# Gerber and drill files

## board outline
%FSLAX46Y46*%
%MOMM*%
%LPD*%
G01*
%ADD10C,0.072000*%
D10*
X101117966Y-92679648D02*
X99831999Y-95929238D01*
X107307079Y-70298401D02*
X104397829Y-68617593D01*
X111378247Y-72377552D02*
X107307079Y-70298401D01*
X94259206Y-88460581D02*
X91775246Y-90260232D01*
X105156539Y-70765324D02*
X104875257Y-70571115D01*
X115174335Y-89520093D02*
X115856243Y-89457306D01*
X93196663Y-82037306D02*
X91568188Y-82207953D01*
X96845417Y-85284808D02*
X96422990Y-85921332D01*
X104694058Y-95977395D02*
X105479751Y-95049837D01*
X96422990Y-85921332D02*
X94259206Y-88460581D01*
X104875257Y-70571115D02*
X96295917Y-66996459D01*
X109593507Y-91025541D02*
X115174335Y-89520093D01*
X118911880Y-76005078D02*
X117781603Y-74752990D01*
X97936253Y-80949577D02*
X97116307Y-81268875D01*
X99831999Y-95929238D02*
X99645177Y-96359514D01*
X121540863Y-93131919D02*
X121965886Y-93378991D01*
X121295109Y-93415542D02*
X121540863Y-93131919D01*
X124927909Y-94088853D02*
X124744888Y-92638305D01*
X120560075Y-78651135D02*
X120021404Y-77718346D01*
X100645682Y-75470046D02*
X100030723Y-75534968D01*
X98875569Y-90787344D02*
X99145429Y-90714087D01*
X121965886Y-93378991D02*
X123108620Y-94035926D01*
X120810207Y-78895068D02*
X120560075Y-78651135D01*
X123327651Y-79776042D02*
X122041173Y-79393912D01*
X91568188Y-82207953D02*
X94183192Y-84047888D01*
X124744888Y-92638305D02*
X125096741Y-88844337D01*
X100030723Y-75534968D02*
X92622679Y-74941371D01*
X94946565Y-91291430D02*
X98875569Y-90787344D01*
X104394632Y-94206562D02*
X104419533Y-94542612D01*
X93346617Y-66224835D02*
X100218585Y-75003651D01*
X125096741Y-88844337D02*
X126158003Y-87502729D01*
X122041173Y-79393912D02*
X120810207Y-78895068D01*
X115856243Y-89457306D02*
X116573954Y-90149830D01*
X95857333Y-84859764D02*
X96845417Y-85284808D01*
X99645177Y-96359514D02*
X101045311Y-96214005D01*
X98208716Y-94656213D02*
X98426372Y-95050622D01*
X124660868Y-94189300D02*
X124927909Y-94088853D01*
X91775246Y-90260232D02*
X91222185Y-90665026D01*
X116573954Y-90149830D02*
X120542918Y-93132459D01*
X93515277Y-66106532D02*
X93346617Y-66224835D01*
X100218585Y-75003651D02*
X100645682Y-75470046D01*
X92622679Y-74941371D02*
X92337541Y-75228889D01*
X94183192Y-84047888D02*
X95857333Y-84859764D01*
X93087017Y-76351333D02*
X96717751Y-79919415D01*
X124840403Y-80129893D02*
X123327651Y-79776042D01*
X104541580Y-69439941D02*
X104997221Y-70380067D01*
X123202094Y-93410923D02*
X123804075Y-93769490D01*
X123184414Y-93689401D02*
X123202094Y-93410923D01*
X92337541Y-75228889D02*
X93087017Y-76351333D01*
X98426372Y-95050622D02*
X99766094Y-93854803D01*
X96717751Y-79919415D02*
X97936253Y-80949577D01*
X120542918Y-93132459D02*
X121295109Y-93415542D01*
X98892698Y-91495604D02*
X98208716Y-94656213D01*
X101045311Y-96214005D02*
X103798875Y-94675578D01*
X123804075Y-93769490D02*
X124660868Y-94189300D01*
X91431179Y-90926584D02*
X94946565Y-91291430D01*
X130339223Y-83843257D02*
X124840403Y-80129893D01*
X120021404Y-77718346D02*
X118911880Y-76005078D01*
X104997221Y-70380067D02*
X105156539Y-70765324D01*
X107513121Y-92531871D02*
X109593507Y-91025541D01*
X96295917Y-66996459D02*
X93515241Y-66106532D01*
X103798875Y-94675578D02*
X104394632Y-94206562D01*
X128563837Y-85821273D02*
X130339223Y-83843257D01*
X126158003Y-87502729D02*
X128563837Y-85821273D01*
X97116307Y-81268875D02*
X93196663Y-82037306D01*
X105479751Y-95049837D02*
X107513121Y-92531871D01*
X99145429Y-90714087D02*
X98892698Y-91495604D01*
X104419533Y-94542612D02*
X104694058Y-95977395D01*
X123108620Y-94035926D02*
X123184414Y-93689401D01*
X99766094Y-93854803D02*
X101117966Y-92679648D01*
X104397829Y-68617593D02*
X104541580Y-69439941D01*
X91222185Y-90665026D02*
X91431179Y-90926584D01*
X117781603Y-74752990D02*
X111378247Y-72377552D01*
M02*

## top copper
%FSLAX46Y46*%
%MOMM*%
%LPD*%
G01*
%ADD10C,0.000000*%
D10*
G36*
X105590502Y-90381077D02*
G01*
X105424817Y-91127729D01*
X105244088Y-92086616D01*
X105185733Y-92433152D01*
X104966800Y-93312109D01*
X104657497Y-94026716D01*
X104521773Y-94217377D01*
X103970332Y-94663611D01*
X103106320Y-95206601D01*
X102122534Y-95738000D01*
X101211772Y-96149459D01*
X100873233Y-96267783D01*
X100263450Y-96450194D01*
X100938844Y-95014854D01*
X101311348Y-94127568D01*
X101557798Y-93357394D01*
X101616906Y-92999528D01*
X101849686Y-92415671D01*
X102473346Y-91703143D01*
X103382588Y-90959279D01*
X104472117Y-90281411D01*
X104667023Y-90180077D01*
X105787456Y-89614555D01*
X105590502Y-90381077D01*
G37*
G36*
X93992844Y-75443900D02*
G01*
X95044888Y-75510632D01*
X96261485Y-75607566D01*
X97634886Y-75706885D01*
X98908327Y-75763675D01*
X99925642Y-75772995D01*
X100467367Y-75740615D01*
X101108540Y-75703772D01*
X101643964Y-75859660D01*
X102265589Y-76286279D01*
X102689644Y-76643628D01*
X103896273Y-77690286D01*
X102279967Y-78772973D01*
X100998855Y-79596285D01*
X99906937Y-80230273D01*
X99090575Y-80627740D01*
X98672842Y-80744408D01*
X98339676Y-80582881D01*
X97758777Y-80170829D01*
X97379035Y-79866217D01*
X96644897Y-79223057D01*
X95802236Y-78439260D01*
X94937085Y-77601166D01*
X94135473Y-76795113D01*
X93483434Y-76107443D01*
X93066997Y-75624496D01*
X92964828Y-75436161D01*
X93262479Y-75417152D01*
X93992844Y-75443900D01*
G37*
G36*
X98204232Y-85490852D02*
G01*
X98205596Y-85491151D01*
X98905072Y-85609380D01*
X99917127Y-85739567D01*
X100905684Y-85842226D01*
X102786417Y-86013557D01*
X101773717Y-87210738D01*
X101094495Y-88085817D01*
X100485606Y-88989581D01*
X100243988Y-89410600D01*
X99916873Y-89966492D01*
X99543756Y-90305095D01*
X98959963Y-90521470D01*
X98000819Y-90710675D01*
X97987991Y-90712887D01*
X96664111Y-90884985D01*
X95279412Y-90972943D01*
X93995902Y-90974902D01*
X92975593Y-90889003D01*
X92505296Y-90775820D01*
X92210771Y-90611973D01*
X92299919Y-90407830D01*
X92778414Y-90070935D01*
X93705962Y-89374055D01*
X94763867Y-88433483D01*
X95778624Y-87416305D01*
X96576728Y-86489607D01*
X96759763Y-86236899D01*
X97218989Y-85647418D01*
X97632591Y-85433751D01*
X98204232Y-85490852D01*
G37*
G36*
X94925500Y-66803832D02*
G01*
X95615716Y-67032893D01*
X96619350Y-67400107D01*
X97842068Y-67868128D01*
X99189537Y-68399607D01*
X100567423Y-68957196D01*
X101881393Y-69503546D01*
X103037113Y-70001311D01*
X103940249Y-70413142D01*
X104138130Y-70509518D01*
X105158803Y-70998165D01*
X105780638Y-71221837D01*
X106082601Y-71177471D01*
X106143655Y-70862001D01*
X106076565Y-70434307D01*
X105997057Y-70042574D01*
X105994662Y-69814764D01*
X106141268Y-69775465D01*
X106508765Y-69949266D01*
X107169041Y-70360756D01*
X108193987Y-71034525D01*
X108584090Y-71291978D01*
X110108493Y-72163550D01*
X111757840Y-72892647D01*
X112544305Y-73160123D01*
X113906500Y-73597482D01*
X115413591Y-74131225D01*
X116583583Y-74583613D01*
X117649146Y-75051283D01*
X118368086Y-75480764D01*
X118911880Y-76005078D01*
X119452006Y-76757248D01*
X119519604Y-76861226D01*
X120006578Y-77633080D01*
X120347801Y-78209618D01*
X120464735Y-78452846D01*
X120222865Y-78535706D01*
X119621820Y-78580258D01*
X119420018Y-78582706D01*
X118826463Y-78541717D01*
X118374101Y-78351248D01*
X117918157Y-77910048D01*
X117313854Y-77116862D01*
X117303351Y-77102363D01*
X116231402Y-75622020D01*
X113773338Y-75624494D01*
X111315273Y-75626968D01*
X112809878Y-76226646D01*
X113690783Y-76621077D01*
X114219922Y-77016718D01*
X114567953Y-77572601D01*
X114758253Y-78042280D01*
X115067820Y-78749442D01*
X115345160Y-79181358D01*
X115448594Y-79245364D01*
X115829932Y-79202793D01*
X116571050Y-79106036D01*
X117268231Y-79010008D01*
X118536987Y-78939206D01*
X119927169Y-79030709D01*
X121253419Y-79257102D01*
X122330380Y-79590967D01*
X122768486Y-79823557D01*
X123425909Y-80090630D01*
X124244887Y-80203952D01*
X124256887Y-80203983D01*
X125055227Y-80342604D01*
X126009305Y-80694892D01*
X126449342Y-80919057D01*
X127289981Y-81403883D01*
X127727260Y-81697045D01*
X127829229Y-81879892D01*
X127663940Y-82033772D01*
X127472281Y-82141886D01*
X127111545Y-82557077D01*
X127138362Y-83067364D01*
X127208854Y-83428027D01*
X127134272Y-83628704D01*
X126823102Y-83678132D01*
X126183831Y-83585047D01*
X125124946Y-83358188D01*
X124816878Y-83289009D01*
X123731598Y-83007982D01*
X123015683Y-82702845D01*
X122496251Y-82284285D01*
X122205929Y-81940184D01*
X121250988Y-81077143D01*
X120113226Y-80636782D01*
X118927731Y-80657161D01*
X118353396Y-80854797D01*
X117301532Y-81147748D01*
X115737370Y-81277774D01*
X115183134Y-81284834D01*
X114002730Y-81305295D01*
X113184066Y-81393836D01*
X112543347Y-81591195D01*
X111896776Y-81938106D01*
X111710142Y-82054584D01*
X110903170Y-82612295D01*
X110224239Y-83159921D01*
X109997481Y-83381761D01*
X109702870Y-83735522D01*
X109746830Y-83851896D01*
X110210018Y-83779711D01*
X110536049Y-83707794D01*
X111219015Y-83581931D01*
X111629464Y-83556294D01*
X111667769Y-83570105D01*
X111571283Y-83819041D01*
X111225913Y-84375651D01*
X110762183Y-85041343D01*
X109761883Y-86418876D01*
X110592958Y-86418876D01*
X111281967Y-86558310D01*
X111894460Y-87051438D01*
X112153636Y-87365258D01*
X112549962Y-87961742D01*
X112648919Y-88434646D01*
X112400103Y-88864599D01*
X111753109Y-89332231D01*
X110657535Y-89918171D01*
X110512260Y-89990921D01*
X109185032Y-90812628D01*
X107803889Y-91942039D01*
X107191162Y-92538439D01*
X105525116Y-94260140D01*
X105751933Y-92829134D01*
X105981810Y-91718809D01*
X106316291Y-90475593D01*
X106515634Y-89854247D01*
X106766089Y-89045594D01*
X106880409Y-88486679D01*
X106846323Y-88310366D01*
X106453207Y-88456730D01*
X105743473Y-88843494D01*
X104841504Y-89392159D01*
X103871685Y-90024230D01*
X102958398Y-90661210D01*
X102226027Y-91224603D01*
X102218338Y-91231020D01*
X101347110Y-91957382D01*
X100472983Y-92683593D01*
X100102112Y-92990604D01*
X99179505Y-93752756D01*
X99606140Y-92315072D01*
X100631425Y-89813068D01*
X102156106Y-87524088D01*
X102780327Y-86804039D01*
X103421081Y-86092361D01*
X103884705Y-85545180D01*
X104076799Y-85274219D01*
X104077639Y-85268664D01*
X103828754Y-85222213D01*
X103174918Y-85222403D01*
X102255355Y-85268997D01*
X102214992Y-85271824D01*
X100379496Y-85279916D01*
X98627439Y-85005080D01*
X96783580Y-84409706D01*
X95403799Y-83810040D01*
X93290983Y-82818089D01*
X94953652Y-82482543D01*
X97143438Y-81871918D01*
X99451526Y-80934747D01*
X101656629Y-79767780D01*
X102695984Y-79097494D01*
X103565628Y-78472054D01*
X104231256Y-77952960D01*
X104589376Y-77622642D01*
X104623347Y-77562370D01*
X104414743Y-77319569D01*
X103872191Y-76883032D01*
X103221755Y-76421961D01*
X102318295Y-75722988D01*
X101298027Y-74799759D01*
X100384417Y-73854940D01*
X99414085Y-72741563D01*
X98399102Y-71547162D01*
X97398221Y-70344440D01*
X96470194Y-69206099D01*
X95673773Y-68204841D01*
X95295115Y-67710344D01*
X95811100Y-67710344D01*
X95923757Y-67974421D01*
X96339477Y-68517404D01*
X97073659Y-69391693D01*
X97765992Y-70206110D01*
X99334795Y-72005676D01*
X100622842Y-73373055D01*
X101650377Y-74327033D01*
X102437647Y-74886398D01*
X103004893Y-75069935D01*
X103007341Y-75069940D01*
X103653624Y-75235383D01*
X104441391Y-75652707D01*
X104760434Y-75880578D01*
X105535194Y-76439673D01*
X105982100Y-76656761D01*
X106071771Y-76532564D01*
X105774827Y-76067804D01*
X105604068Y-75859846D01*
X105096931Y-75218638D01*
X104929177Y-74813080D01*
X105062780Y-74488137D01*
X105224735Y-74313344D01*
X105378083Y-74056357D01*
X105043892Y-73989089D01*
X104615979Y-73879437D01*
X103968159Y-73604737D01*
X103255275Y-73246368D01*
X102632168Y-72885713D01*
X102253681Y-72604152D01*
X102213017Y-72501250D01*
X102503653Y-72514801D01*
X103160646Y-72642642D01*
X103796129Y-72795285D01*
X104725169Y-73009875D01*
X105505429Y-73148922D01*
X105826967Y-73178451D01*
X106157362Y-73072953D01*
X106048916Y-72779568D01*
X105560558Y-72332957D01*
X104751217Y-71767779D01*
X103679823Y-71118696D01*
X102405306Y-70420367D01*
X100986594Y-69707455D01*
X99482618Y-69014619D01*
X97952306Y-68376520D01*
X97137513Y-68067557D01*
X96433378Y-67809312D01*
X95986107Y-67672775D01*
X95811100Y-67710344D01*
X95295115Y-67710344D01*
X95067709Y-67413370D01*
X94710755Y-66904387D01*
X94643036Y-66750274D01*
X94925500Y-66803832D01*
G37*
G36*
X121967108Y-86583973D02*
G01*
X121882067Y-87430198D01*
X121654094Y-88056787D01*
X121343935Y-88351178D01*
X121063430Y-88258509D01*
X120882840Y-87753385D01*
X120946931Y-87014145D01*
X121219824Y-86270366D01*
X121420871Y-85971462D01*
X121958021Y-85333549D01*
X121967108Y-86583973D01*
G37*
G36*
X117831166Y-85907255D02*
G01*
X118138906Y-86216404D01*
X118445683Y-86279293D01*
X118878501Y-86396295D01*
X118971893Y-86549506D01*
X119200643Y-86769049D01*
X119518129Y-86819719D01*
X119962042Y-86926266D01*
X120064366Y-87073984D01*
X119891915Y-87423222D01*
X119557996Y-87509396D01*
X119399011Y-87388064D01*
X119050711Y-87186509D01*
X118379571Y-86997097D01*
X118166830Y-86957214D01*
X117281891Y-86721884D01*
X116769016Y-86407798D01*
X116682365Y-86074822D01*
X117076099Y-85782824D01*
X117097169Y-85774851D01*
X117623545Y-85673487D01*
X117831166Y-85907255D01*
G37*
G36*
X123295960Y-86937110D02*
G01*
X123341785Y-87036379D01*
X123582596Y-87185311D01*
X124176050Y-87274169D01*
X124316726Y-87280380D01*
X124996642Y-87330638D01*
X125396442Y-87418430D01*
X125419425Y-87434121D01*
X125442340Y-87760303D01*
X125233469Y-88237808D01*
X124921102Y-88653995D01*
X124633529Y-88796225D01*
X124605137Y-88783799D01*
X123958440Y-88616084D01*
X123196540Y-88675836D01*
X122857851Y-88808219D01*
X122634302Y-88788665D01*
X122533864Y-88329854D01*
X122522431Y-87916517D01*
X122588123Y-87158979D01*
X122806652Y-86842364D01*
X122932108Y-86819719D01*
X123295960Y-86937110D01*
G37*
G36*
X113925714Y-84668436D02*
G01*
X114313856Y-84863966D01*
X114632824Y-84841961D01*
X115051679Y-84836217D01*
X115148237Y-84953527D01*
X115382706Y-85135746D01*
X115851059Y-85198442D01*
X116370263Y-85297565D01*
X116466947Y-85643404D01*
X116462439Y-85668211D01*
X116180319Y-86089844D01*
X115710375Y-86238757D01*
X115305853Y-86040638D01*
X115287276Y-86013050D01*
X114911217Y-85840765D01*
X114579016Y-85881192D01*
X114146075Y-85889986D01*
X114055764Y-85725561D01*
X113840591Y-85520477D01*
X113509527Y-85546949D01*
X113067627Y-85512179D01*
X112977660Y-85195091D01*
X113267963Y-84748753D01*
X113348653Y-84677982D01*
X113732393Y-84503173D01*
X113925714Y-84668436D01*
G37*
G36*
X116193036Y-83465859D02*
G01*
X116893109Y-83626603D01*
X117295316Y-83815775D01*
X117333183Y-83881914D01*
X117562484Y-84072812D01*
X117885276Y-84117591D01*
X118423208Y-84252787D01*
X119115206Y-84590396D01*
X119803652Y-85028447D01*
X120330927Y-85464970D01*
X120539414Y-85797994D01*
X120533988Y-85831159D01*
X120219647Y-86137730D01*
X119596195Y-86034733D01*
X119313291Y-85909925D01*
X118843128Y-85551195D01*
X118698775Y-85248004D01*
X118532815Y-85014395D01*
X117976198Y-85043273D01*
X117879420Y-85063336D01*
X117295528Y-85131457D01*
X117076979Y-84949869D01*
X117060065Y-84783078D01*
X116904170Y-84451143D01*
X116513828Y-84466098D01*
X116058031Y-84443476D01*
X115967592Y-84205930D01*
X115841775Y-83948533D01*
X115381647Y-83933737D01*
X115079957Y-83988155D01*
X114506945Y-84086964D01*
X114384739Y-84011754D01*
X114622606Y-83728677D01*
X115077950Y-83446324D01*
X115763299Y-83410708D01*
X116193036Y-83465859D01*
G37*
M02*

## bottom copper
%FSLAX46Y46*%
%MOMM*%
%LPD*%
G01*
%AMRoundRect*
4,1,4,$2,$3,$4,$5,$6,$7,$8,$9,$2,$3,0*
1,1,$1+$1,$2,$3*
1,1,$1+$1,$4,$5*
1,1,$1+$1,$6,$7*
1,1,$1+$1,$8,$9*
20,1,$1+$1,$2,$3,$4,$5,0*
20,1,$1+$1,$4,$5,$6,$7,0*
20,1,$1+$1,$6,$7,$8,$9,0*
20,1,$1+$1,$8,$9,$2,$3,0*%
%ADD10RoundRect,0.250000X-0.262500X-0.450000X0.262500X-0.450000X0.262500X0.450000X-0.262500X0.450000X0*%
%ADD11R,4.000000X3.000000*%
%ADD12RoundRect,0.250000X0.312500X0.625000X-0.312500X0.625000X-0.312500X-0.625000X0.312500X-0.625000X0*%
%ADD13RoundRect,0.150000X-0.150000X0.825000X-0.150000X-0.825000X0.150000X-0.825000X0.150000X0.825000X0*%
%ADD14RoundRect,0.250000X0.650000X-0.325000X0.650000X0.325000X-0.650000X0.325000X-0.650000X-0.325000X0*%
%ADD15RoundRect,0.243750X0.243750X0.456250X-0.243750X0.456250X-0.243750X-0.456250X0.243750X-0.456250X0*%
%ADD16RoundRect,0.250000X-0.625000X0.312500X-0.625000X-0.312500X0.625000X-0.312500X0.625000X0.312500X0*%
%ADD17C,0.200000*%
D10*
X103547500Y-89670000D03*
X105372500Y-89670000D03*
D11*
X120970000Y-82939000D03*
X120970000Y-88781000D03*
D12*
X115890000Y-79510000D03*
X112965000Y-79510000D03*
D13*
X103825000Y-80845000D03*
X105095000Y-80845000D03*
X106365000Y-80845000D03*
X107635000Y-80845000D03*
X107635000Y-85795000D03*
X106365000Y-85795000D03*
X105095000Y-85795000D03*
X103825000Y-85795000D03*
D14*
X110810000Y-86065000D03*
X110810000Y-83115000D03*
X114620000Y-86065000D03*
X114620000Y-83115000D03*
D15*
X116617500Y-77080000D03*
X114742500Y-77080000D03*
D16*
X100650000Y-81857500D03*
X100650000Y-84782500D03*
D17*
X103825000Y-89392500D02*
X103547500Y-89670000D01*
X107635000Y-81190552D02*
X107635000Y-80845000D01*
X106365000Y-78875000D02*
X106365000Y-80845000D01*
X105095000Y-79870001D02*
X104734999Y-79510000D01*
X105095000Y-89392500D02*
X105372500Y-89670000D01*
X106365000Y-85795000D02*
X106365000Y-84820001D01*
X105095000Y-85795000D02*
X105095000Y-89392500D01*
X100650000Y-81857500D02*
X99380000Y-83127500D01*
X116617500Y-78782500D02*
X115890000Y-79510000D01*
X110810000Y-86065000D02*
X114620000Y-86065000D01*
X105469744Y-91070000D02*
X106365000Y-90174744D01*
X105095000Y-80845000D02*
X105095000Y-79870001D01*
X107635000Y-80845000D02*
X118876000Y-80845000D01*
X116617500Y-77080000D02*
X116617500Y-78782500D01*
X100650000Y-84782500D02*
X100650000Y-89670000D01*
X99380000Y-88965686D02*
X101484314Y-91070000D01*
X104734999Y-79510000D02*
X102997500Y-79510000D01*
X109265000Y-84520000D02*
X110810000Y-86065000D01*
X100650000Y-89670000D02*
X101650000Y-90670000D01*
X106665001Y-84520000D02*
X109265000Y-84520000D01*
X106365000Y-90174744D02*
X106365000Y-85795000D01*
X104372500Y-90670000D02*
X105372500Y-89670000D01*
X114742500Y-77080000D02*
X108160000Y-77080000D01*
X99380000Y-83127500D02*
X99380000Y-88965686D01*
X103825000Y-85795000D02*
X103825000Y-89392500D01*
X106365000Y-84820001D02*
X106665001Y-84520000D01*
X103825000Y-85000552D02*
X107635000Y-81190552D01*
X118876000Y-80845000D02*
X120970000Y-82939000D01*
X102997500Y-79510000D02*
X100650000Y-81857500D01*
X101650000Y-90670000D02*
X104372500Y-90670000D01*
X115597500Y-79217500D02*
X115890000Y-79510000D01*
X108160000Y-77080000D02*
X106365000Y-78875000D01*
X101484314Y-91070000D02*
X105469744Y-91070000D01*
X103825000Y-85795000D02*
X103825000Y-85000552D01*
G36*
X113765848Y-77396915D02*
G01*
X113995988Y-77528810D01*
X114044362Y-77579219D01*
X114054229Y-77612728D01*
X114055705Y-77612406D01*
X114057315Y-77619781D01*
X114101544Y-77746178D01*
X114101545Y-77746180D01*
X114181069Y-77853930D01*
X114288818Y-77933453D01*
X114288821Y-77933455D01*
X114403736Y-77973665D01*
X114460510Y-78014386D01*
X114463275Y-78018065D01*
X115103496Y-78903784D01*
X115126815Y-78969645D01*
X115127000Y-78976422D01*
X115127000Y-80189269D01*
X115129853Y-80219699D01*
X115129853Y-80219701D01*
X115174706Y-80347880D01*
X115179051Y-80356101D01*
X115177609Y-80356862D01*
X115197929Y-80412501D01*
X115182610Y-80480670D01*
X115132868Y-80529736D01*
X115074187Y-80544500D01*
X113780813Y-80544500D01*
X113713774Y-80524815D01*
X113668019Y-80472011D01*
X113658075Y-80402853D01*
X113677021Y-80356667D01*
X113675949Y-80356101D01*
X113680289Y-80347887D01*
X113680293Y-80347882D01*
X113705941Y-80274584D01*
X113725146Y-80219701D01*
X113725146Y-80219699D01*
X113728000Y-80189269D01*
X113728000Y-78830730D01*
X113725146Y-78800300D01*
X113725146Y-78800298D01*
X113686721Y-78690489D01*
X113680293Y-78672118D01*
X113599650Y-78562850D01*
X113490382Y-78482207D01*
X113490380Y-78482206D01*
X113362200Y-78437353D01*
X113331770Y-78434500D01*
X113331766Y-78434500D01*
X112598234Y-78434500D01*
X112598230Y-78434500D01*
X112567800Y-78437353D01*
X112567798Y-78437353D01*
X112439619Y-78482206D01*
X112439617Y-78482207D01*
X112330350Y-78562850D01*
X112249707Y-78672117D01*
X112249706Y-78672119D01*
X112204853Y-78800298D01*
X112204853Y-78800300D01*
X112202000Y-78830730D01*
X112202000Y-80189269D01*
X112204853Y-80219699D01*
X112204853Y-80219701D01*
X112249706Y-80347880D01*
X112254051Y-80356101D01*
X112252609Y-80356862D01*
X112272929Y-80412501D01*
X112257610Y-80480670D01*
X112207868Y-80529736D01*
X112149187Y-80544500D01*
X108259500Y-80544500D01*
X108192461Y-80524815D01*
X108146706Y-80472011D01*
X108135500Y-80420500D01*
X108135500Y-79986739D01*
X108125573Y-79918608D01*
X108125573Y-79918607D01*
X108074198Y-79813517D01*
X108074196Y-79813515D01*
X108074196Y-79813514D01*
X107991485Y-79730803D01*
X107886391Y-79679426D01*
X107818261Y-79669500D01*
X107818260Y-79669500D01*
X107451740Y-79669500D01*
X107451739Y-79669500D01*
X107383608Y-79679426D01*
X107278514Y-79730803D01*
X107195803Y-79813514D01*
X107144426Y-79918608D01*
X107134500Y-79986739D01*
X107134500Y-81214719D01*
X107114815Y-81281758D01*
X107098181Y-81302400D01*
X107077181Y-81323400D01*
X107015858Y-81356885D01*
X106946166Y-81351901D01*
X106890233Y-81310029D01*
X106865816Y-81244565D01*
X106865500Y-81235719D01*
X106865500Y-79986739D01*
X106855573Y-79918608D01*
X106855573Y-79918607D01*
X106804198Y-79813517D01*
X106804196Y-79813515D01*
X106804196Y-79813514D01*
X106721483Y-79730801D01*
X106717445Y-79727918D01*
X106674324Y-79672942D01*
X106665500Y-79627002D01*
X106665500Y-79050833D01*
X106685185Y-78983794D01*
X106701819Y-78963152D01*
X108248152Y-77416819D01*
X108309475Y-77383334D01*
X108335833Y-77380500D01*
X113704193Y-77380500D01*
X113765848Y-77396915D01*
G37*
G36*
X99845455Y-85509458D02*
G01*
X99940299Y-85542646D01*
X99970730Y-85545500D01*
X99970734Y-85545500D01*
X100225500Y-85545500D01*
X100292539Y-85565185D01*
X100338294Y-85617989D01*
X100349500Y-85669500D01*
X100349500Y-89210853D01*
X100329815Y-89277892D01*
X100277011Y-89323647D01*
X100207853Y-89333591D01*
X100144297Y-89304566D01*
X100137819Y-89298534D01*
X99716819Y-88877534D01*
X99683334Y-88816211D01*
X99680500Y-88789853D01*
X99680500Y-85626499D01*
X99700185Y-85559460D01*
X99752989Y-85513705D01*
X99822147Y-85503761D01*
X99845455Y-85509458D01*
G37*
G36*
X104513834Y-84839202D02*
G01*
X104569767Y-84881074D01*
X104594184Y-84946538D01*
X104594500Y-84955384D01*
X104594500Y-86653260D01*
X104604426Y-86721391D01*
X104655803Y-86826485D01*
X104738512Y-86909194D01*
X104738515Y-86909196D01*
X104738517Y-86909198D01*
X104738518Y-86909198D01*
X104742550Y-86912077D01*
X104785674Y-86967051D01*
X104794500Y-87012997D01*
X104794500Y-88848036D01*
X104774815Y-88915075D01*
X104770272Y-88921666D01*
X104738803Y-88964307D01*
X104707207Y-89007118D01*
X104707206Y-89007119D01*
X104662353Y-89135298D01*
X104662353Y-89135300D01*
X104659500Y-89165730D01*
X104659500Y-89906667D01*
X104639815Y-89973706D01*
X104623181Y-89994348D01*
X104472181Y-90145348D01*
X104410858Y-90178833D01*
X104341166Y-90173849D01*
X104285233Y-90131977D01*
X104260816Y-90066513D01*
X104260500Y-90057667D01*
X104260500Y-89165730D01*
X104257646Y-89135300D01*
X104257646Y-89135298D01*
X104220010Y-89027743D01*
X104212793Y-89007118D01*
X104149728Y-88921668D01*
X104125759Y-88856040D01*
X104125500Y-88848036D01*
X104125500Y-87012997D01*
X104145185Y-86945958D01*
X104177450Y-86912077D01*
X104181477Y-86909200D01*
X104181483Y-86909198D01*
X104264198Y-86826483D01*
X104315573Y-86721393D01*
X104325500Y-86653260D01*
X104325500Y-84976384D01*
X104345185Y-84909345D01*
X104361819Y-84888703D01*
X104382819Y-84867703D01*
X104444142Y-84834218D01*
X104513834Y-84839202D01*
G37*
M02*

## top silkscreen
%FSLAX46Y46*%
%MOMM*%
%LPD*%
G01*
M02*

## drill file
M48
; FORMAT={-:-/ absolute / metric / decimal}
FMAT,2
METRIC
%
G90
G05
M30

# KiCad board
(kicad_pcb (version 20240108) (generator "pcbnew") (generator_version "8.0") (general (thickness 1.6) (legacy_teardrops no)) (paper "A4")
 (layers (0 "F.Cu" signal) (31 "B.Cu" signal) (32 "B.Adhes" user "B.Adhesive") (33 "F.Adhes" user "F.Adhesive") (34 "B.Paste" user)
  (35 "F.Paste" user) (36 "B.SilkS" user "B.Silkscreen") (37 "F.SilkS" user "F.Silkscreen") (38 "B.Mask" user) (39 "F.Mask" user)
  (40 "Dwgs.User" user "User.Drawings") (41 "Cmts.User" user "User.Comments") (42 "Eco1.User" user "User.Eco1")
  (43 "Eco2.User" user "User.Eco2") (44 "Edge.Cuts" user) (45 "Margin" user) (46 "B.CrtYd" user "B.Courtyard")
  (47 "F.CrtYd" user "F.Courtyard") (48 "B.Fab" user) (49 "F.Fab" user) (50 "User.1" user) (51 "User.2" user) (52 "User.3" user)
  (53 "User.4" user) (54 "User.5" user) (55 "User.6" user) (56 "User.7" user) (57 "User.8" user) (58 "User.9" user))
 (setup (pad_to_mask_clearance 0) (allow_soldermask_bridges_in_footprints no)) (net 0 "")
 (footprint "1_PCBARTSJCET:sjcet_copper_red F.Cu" (layer "F.Cu") (at 118.552907 138.299727)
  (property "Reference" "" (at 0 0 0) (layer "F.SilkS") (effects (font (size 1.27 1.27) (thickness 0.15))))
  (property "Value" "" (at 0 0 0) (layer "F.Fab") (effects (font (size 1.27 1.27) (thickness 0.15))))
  (fp_poly
   (pts (xy -12.962405 -47.91865) (xy -13.12809 -47.171998) (xy -13.308819 -46.213111) (xy -13.367174 -45.866575) (xy -13.586107 -44.987618)
    (xy -13.89541 -44.273011) (xy -14.031134 -44.08235) (xy -14.582575 -43.636116) (xy -15.446587 -43.093126) (xy -16.430373 -42.561727)
    (xy -17.341135 -42.150268) (xy -17.679674 -42.031944) (xy -18.289457 -41.849533) (xy -17.614063 -43.284873) (xy -17.241559 -44.172159)
    (xy -16.995109 -44.942333) (xy -16.936001 -45.300199) (xy -16.703221 -45.884056) (xy -16.079561 -46.596584) (xy -15.170319 -47.340448)
    (xy -14.08079 -48.018316) (xy -13.885884 -48.11965) (xy -12.765451 -48.685172))
   (stroke (width 0) (type solid)) (fill solid) (layer "F.Cu"))
  (fp_poly
   (pts (xy -24.560063 -62.855827) (xy -23.508019 -62.789095) (xy -22.291422 -62.692161) (xy -20.918021 -62.592842)
    (xy -19.64458 -62.536052) (xy -18.627265 -62.526732) (xy -18.08554 -62.559112) (xy -17.444367 -62.595955) (xy -16.908943 -62.440067)
    (xy -16.287318 -62.013448) (xy -15.863263 -61.656099) (xy -14.656634 -60.609441) (xy -16.27294 -59.526754) (xy -17.554052 -58.703442)
    (xy -18.64597 -58.069454) (xy -19.462332 -57.671987) (xy -19.880065 -57.555319) (xy -20.213231 -57.716846) (xy -20.79413 -58.128898)
    (xy -21.173872 -58.43351) (xy -21.90801 -59.07667) (xy -22.750671 -59.860467) (xy -23.615822 -60.698561) (xy -24.417434 -61.504614)
    (xy -25.069473 -62.192284) (xy -25.48591 -62.675231) (xy -25.588079 -62.863566) (xy -25.290428 -62.882575))
   (stroke (width 0) (type solid)) (fill solid) (layer "F.Cu"))
  (fp_poly
   (pts (xy -20.348675 -52.808875) (xy -20.347311 -52.808576) (xy -19.647835 -52.690347) (xy -18.63578 -52.56016) (xy -17.647223 -52.457501)
    (xy -15.76649 -52.28617) (xy -16.77919 -51.088989) (xy -17.458412 -50.21391) (xy -18.067301 -49.310146) (xy -18.308919 -48.889127)
    (xy -18.636034 -48.333235) (xy -19.009151 -47.994632) (xy -19.592944 -47.778257) (xy -20.552088 -47.589052) (xy -20.564916 -47.58684)
    (xy -21.888796 -47.414742) (xy -23.273495 -47.326784) (xy -24.557005 -47.324825) (xy -25.577314 -47.410724) (xy -26.047611 -47.523907)
    (xy -26.342136 -47.687754) (xy -26.252988 -47.891897) (xy -25.774493 -48.228792) (xy -24.846945 -48.925672) (xy -23.78904 -49.866244)
    (xy -22.774283 -50.883422) (xy -21.976179 -51.81012) (xy -21.793144 -52.062828) (xy -21.333918 -52.652309) (xy -20.920316 -52.865976))
   (stroke (width 0) (type solid)) (fill solid) (layer "F.Cu"))
  (fp_poly
   (pts (xy -23.627407 -71.495895) (xy -22.937191 -71.266834) (xy -21.933557 -70.89962) (xy -20.710839 -70.431599) (xy -19.36337 -69.90012)
    (xy -17.985484 -69.342531) (xy -16.671514 -68.796181) (xy -15.515794 -68.298416) (xy -14.612658 -67.886585) (xy -14.414777 -67.790209)
    (xy -13.394104 -67.301562) (xy -12.772269 -67.07789) (xy -12.470306 -67.122256) (xy -12.409252 -67.437726) (xy -12.476342 -67.86542)
    (xy -12.55585 -68.257153) (xy -12.558245 -68.484963) (xy -12.411639 -68.524262) (xy -12.044142 -68.350461) (xy -11.383866 -67.938971)
    (xy -10.35892 -67.265202) (xy -9.968817 -67.007749) (xy -8.444414 -66.136177) (xy -6.795067 -65.40708) (xy -6.008602 -65.139604)
    (xy -4.646407 -64.702245) (xy -3.139316 -64.168502) (xy -1.969324 -63.716114) (xy -0.903761 -63.248444) (xy -0.184821 -62.818963)
    (xy 0.358973 -62.294649) (xy 0.899099 -61.542479) (xy 0.966697 -61.438501) (xy 1.453671 -60.666647) (xy 1.794894 -60.090109)
    (xy 1.911828 -59.846881) (xy 1.669958 -59.764021) (xy 1.068913 -59.719469) (xy 0.867111 -59.717021) (xy 0.273556 -59.75801)
    (xy -0.178806 -59.948479) (xy -0.63475 -60.389679) (xy -1.239053 -61.182865) (xy -1.249556 -61.197364) (xy -2.321505 -62.677707)
    (xy -4.779569 -62.675233) (xy -7.237634 -62.672759) (xy -5.743029 -62.073081) (xy -4.862124 -61.67865) (xy -4.332985 -61.283009)
    (xy -3.984954 -60.727126) (xy -3.794654 -60.257447) (xy -3.485087 -59.550285) (xy -3.207747 -59.118369) (xy -3.104313 -59.054363)
    (xy -2.722975 -59.096934) (xy -1.981857 -59.193691) (xy -1.284676 -59.289719) (xy -0.01592 -59.360521) (xy 1.374262 -59.269018)
    (xy 2.700512 -59.042625) (xy 3.777473 -58.70876) (xy 4.215579 -58.47617) (xy 4.873002 -58.209097) (xy 5.69198 -58.095775)
    (xy 5.70398 -58.095744) (xy 6.50232 -57.957123) (xy 7.456398 -57.604835) (xy 7.896435 -57.38067) (xy 8.737074 -56.895844)
    (xy 9.174353 -56.602682) (xy 9.276322 -56.419835) (xy 9.111033 -56.265955) (xy 8.919374 -56.157841) (xy 8.558638 -55.74265)
    (xy 8.585455 -55.232363) (xy 8.655947 -54.8717) (xy 8.581365 -54.671023) (xy 8.270195 -54.621595) (xy 7.630924 -54.71468)
    (xy 6.572039 -54.941539) (xy 6.263971 -55.010718) (xy 5.178691 -55.291745) (xy 4.462776 -55.596882) (xy 3.943344 -56.015442)
    (xy 3.653022 -56.359543) (xy 2.698081 -57.222584) (xy 1.560319 -57.662945) (xy 0.374824 -57.642566) (xy -0.199511 -57.44493)
    (xy -1.251375 -57.151979) (xy -2.815537 -57.021953) (xy -3.369773 -57.014893) (xy -4.550177 -56.994432) (xy -5.368841 -56.905891)
    (xy -6.00956 -56.708532) (xy -6.656131 -56.361621) (xy -6.842765 -56.245143) (xy -7.649737 -55.687432) (xy -8.328668 -55.139806)
    (xy -8.555426 -54.917966) (xy -8.850037 -54.564205) (xy -8.806077 -54.447831) (xy -8.342889 -54.520016) (xy -8.016858 -54.591933)
    (xy -7.333892 -54.717796) (xy -6.923443 -54.743433) (xy -6.885138 -54.729622) (xy -6.981624 -54.480686) (xy -7.326994 -53.924076)
    (xy -7.790724 -53.258384) (xy -8.791024 -51.880851) (xy -7.959949 -51.880851) (xy -7.27094 -51.741417) (xy -6.658447 -51.248289)
    (xy -6.399271 -50.934469) (xy -6.002945 -50.337985) (xy -5.903988 -49.865081) (xy -6.152804 -49.435128) (xy -6.799798 -48.967496)
    (xy -7.895372 -48.381556) (xy -8.040647 -48.308806) (xy -9.367875 -47.487099) (xy -10.749018 -46.357688) (xy -11.361745 -45.761288)
    (xy -13.027791 -44.039587) (xy -12.800974 -45.470593) (xy -12.571097 -46.580918) (xy -12.236616 -47.824134) (xy -12.037273 -48.44548)
    (xy -11.786818 -49.254133) (xy -11.672498 -49.813048) (xy -11.706584 -49.989361) (xy -12.0997 -49.842997) (xy -12.809434 -49.456233)
    (xy -13.711403 -48.907568) (xy -14.681222 -48.275497) (xy -15.594509 -47.638517) (xy -16.32688 -47.075124) (xy -16.334569 -47.068707)
    (xy -17.205797 -46.342345) (xy -18.079924 -45.616134) (xy -18.450795 -45.309123) (xy -19.373402 -44.546971) (xy -18.946767 -45.984655)
    (xy -17.921482 -48.486659) (xy -16.396801 -50.775639) (xy -15.77258 -51.495688) (xy -15.131826 -52.207366) (xy -14.668202 -52.754547)
    (xy -14.476108 -53.025508) (xy -14.475268 -53.031063) (xy -14.724153 -53.077514) (xy -15.377989 -53.077324) (xy -16.297552 -53.03073)
    (xy -16.337915 -53.027903) (xy -18.173411 -53.019811) (xy -19.925468 -53.294647) (xy -21.769327 -53.890021) (xy -23.149108 -54.489687)
    (xy -25.261924 -55.481638) (xy -23.599255 -55.817184) (xy -21.409469 -56.427809) (xy -19.101381 -57.36498) (xy -16.896278 -58.531947)
    (xy -15.856923 -59.202233) (xy -14.987279 -59.827673) (xy -14.321651 -60.346767) (xy -13.963531 -60.677085) (xy -13.92956 -60.737357)
    (xy -14.138164 -60.980158) (xy -14.680716 -61.416695) (xy -15.331152 -61.877766) (xy -16.234612 -62.576739) (xy -17.25488 -63.499968)
    (xy -18.16849 -64.444787) (xy -19.138822 -65.558164) (xy -20.153805 -66.752565) (xy -21.154686 -67.955287) (xy -22.082713 -69.093628)
    (xy -22.879134 -70.094886) (xy -23.257792 -70.589383) (xy -22.741807 -70.589383) (xy -22.62915 -70.325306) (xy -22.21343 -69.782323)
    (xy -21.479248 -68.908034) (xy -20.786915 -68.093617) (xy -19.218112 -66.294051) (xy -17.930065 -64.926672) (xy -16.90253 -63.972694)
    (xy -16.11526 -63.413329) (xy -15.548014 -63.229792) (xy -15.545566 -63.229787) (xy -14.899283 -63.064344) (xy -14.111516 -62.64702)
    (xy -13.792473 -62.419149) (xy -13.017713 -61.860054) (xy -12.570807 -61.642966) (xy -12.481136 -61.767163) (xy -12.77808 -62.231923)
    (xy -12.948839 -62.439881) (xy -13.455976 -63.081089) (xy -13.62373 -63.486647) (xy -13.490127 -63.81159) (xy -13.328172 -63.986383)
    (xy -13.174824 -64.24337) (xy -13.509015 -64.310638) (xy -13.936928 -64.42029) (xy -14.584748 -64.69499) (xy -15.297632 -65.053359)
    (xy -15.920739 -65.414014) (xy -16.299226 -65.695575) (xy -16.33989 -65.798477) (xy -16.049254 -65.784926) (xy -15.392261 -65.657085)
    (xy -14.756778 -65.504442) (xy -13.827738 -65.289852) (xy -13.047478 -65.150805) (xy -12.72594 -65.121276) (xy -12.395545 -65.226774)
    (xy -12.503991 -65.520159) (xy -12.992349 -65.96677) (xy -13.80169 -66.531948) (xy -14.873084 -67.181031) (xy -16.147601 -67.87936)
    (xy -17.566313 -68.592272) (xy -19.070289 -69.285108) (xy -20.600601 -69.923207) (xy -21.415394 -70.23217) (xy -22.119529 -70.490415)
    (xy -22.5668 -70.626952) (xy -22.741807 -70.589383) (xy -23.257792 -70.589383) (xy -23.485198 -70.886357) (xy -23.842152 -71.39534)
    (xy -23.909871 -71.549453))
   (stroke (width 0) (type solid)) (fill solid) (layer "F.Cu")))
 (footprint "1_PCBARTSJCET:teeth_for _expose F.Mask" (layer "F.Cu") (at 119.618129 137.199293)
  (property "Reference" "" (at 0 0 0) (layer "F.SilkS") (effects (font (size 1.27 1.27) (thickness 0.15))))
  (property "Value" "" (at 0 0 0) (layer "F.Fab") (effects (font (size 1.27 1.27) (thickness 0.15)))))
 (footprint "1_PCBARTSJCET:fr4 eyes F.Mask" (layer "F.Cu") (at 125.66 135.17)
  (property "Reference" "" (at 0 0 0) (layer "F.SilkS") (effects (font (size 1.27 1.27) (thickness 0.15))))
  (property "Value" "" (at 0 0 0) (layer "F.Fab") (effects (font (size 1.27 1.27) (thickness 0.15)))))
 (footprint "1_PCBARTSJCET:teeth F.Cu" (layer "F.Cu") (at 119.518129 137.079293)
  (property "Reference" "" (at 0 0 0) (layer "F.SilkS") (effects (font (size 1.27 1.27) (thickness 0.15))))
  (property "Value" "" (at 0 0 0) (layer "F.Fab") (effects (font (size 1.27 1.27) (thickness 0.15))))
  (fp_poly
   (pts (xy 2.448979 -50.49532) (xy 2.363938 -49.649095) (xy 2.135965 -49.022506) (xy 1.825806 -48.728115) (xy 1.545301 -48.820784)
    (xy 1.364711 -49.325908) (xy 1.428802 -50.065148) (xy 1.701695 -50.808927) (xy 1.902742 -51.107831) (xy 2.439892 -51.745744))
   (stroke (width 0) (type solid)) (fill solid) (layer "F.Cu"))
  (fp_poly
   (pts (xy -1.686963 -51.172038) (xy -1.379223 -50.862889) (xy -1.072446 -50.8) (xy -0.639628 -50.682998) (xy -0.546236 -50.529787)
    (xy -0.317486 -50.310244) (xy 0 -50.259574) (xy 0.443913 -50.153027) (xy 0.546237 -50.005309) (xy 0.373786 -49.656071)
    (xy 0.039867 -49.569897) (xy -0.119118 -49.691229) (xy -0.467418 -49.892784) (xy -1.138558 -50.082196) (xy -1.351299 -50.122079)
    (xy -2.236238 -50.357409) (xy -2.749113 -50.671495) (xy -2.835764 -51.004471) (xy -2.44203 -51.296469) (xy -2.42096 -51.304442)
    (xy -1.894584 -51.405806))
   (stroke (width 0) (type solid)) (fill solid) (layer "F.Cu"))
  (fp_poly
   (pts (xy 3.777831 -50.142183) (xy 3.823656 -50.042914) (xy 4.064467 -49.893982) (xy 4.657921 -49.805124) (xy 4.798597 -49.798913)
    (xy 5.478513 -49.748655) (xy 5.878313 -49.660863) (xy 5.901296 -49.645172) (xy 5.924211 -49.31899) (xy 5.71534 -48.841485)
    (xy 5.402973 -48.425298) (xy 5.1154 -48.283068) (xy 5.087008 -48.295494) (xy 4.440311 -48.463209) (xy 3.678411 -48.403457)
    (xy 3.339722 -48.271074) (xy 3.116173 -48.290628) (xy 3.015735 -48.749439) (xy 3.004302 -49.162776) (xy 3.069994 -49.920314)
    (xy 3.288523 -50.236929) (xy 3.413979 -50.259574))
   (stroke (width 0) (type solid)) (fill solid) (layer "F.Cu"))
  (fp_poly
   (pts (xy -5.592415 -52.410857) (xy -5.204273 -52.215327) (xy -4.885305 -52.237332) (xy -4.46645 -52.243076) (xy -4.369892 -52.125766)
    (xy -4.135423 -51.943547) (xy -3.66707 -51.880851) (xy -3.147866 -51.781728) (xy -3.051182 -51.435889) (xy -3.05569 -51.411082)
    (xy -3.33781 -50.989449) (xy -3.807754 -50.840536) (xy -4.212276 -51.038655) (xy -4.230853 -51.066243) (xy -4.606912 -51.238528)
    (xy -4.939113 -51.198101) (xy -5.372054 -51.189307) (xy -5.462365 -51.353732) (xy -5.677538 -51.558816) (xy -6.008602 -51.532344)
    (xy -6.450502 -51.567114) (xy -6.540469 -51.884202) (xy -6.250166 -52.33054) (xy -6.169476 -52.401311) (xy -5.785736 -52.57612))
   (stroke (width 0) (type solid)) (fill solid) (layer "F.Cu"))
  (fp_poly
   (pts (xy -3.325093 -53.613434) (xy -2.62502 -53.45269) (xy -2.222813 -53.263518) (xy -2.184946 -53.197379) (xy -1.955645 -53.006481)
    (xy -1.632853 -52.961702) (xy -1.094921 -52.826506) (xy -0.402923 -52.488897) (xy 0.285523 -52.050846) (xy 0.812798 -51.614323)
    (xy 1.021285 -51.281299) (xy 1.015859 -51.248134) (xy 0.701518 -50.941563) (xy 0.078066 -51.04456) (xy -0.204838 -51.169368)
    (xy -0.675001 -51.528098) (xy -0.819354 -51.831289) (xy -0.985314 -52.064898) (xy -1.541931 -52.03602) (xy -1.638709 -52.015957)
    (xy -2.222601 -51.947836) (xy -2.44115 -52.129424) (xy -2.458064 -52.296215) (xy -2.613959 -52.62815) (xy -3.004301 -52.613195)
    (xy -3.460098 -52.635817) (xy -3.550537 -52.873363) (xy -3.676354 -53.13076) (xy -4.136482 -53.145556) (xy -4.438172 -53.091138)
    (xy -5.011184 -52.992329) (xy -5.13339 -53.067539) (xy -4.895523 -53.350616) (xy -4.440179 -53.632969) (xy -3.75483 -53.668585))
   (stroke (width 0) (type solid)) (fill solid) (layer "F.Cu")))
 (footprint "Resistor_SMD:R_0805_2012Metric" (layer "B.Cu") (at 104.46 89.67)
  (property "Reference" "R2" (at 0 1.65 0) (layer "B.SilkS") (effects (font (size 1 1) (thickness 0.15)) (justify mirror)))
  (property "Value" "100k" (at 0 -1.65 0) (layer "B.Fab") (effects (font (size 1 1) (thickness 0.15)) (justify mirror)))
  (pad "1" smd roundrect (at -0.9125 0) (size 1.025 1.4) (layers "B.Cu" "B.Paste" "B.Mask") (roundrect_rratio 0.243902))
  (pad "2" smd roundrect (at 0.9125 0) (size 1.025 1.4) (layers "B.Cu" "B.Paste" "B.Mask") (roundrect_rratio 0.243902)))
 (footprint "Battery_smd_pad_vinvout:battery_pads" (layer "B.Cu") (at 113.35 85.225 -90)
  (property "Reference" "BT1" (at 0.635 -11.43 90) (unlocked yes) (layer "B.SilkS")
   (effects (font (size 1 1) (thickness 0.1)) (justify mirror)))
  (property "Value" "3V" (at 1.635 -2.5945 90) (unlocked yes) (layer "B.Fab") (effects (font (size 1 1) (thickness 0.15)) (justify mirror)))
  (pad "1" smd rect (at -2.286 -7.62 270) (size 3 4) (layers "B.Cu" "B.Paste" "B.Mask"))
  (pad "2" smd rect (at 3.556 -7.62 270) (size 3 4) (layers "B.Cu" "B.Paste" "B.Mask")))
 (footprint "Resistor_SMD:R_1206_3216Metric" (layer "B.Cu") (at 114.4275 79.51 180)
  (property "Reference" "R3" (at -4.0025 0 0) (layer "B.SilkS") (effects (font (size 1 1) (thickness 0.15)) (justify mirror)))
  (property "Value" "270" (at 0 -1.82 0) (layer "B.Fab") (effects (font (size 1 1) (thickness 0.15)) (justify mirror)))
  (pad "1" smd roundrect (at -1.4625 0 180) (size 1.125 1.75) (layers "B.Cu" "B.Paste" "B.Mask") (roundrect_rratio 0.222222))
  (pad "2" smd roundrect (at 1.4625 0 180) (size 1.125 1.75) (layers "B.Cu" "B.Paste" "B.Mask") (roundrect_rratio 0.222222)))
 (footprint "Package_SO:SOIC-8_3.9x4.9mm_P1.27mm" (layer "B.Cu") (at 105.73 83.32 -90)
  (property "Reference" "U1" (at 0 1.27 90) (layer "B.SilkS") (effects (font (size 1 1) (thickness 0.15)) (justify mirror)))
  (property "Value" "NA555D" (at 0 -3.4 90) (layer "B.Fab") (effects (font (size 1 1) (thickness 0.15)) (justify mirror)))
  (pad "1" smd roundrect (at -2.475 1.905 270) (size 1.95 0.6) (layers "B.Cu" "B.Paste" "B.Mask") (roundrect_rratio 0.25))
  (pad "2" smd roundrect (at -2.475 0.635 270) (size 1.95 0.6) (layers "B.Cu" "B.Paste" "B.Mask") (roundrect_rratio 0.25))
  (pad "3" smd roundrect (at -2.475 -0.635 270) (size 1.95 0.6) (layers "B.Cu" "B.Paste" "B.Mask") (roundrect_rratio 0.25))
  (pad "4" smd roundrect (at -2.475 -1.905 270) (size 1.95 0.6) (layers "B.Cu" "B.Paste" "B.Mask") (roundrect_rratio 0.25))
  (pad "5" smd roundrect (at 2.475 -1.905 270) (size 1.95 0.6) (layers "B.Cu" "B.Paste" "B.Mask") (roundrect_rratio 0.25))
  (pad "6" smd roundrect (at 2.475 -0.635 270) (size 1.95 0.6) (layers "B.Cu" "B.Paste" "B.Mask") (roundrect_rratio 0.25))
  (pad "7" smd roundrect (at 2.475 0.635 270) (size 1.95 0.6) (layers "B.Cu" "B.Paste" "B.Mask") (roundrect_rratio 0.25))
  (pad "8" smd roundrect (at 2.475 1.905 270) (size 1.95 0.6) (layers "B.Cu" "B.Paste" "B.Mask") (roundrect_rratio 0.25)))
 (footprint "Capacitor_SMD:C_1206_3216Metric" (layer "B.Cu") (at 110.81 84.59 90)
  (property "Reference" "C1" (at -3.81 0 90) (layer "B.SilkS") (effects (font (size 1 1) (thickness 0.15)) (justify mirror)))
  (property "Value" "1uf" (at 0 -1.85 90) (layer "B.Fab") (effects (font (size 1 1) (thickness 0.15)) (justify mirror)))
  (pad "1" smd roundrect (at -1.475 0 90) (size 1.15 1.8) (layers "B.Cu" "B.Paste" "B.Mask") (roundrect_rratio 0.217391))
  (pad "2" smd roundrect (at 1.475 0 90) (size 1.15 1.8) (layers "B.Cu" "B.Paste" "B.Mask") (roundrect_rratio 0.217391)))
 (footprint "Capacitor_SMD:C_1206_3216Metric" (layer "B.Cu") (at 114.62 84.59 90)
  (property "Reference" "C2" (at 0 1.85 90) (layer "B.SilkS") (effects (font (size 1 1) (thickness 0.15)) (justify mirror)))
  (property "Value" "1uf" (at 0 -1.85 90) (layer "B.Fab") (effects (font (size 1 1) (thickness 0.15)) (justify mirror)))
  (pad "1" smd roundrect (at -1.475 0 90) (size 1.15 1.8) (layers "B.Cu" "B.Paste" "B.Mask") (roundrect_rratio 0.217391))
  (pad "2" smd roundrect (at 1.475 0 90) (size 1.15 1.8) (layers "B.Cu" "B.Paste" "B.Mask") (roundrect_rratio 0.217391)))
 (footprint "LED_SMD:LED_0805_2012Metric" (layer "B.Cu") (at 115.68 77.08 180)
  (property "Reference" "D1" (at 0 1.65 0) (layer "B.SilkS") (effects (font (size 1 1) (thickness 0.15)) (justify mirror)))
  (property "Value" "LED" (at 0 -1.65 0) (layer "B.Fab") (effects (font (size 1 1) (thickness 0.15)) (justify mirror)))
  (pad "1" smd roundrect (at -0.9375 0 180) (size 0.975 1.4) (layers "B.Cu" "B.Paste" "B.Mask") (roundrect_rratio 0.25))
  (pad "2" smd roundrect (at 0.9375 0 180) (size 0.975 1.4) (layers "B.Cu" "B.Paste" "B.Mask") (roundrect_rratio 0.25)))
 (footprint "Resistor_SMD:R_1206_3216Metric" (layer "B.Cu") (at 100.65 83.32 -90)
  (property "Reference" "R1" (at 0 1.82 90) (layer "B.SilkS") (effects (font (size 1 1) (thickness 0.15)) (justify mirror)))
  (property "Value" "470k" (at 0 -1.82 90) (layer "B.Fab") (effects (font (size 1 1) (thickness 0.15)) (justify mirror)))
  (pad "1" smd roundrect (at -1.4625 0 270) (size 1.125 1.75) (layers "B.Cu" "B.Paste" "B.Mask") (roundrect_rratio 0.222222))
  (pad "2" smd roundrect (at 1.4625 0 270) (size 1.125 1.75) (layers "B.Cu" "B.Paste" "B.Mask") (roundrect_rratio 0.222222)))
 (gr_line (start 101.117966 92.679648) (end 99.831999 95.929238) (stroke (width 0.072) (type default)) (layer "Edge.Cuts"))
 (gr_line (start 107.307079 70.298401) (end 104.397829 68.617593) (stroke (width 0.072) (type default)) (layer "Edge.Cuts"))
 (gr_line (start 111.378247 72.377552) (end 107.307079 70.298401) (stroke (width 0.072) (type default)) (layer "Edge.Cuts"))
 (gr_line (start 94.259206 88.460581) (end 91.775246 90.260232) (stroke (width 0.072) (type default)) (layer "Edge.Cuts"))
 (gr_line (start 105.156539 70.765324) (end 104.875257 70.571115) (stroke (width 0.072) (type default)) (layer "Edge.Cuts"))
 (gr_line (start 115.174335 89.520093) (end 115.856243 89.457306) (stroke (width 0.072) (type default)) (layer "Edge.Cuts"))
 (gr_line (start 93.196663 82.037306) (end 91.568188 82.207953) (stroke (width 0.072) (type default)) (layer "Edge.Cuts"))
 (gr_line (start 96.845417 85.284808) (end 96.42299 85.921332) (stroke (width 0.072) (type default)) (layer "Edge.Cuts"))
 (gr_line (start 104.694058 95.977395) (end 105.479751 95.049837) (stroke (width 0.072) (type default)) (layer "Edge.Cuts"))
 (gr_line (start 96.42299 85.921332) (end 94.259206 88.460581) (stroke (width 0.072) (type default)) (layer "Edge.Cuts"))
 (gr_line (start 104.875257 70.571115) (end 96.295917 66.996459) (stroke (width 0.072) (type default)) (layer "Edge.Cuts"))
 (gr_line (start 109.593507 91.025541) (end 115.174335 89.520093) (stroke (width 0.072) (type default)) (layer "Edge.Cuts"))
 (gr_line (start 118.91188 76.005078) (end 117.781603 74.75299) (stroke (width 0.072) (type default)) (layer "Edge.Cuts"))
 (gr_line (start 97.936253 80.949577) (end 97.116307 81.268875) (stroke (width 0.072) (type default)) (layer "Edge.Cuts"))
 (gr_line (start 99.831999 95.929238) (end 99.645177 96.359514) (stroke (width 0.072) (type default)) (layer "Edge.Cuts"))
 (gr_line (start 121.540863 93.131919) (end 121.965886 93.378991) (stroke (width 0.072) (type default)) (layer "Edge.Cuts"))
 (gr_line (start 121.295109 93.415542) (end 121.540863 93.131919) (stroke (width 0.072) (type default)) (layer "Edge.Cuts"))
 (gr_line (start 124.927909 94.088853) (end 124.744888 92.638305) (stroke (width 0.072) (type default)) (layer "Edge.Cuts"))
 (gr_line (start 120.560075 78.651135) (end 120.021404 77.718346) (stroke (width 0.072) (type default)) (layer "Edge.Cuts"))
 (gr_line (start 100.645682 75.470046) (end 100.030723 75.534968) (stroke (width 0.072) (type default)) (layer "Edge.Cuts"))
 (gr_line (start 98.875569 90.787344) (end 99.145429 90.714087) (stroke (width 0.072) (type default)) (layer "Edge.Cuts"))
 (gr_line (start 121.965886 93.378991) (end 123.10862 94.035926) (stroke (width 0.072) (type default)) (layer "Edge.Cuts"))
 (gr_line (start 120.810207 78.895068) (end 120.560075 78.651135) (stroke (width 0.072) (type default)) (layer "Edge.Cuts"))
 (gr_line (start 123.327651 79.776042) (end 122.041173 79.393912) (stroke (width 0.072) (type default)) (layer "Edge.Cuts"))
 (gr_line (start 91.568188 82.207953) (end 94.183192 84.047888) (stroke (width 0.072) (type default)) (layer "Edge.Cuts"))
 (gr_line (start 124.744888 92.638305) (end 125.096741 88.844337) (stroke (width 0.072) (type default)) (layer "Edge.Cuts"))
 (gr_line (start 100.030723 75.534968) (end 92.622679 74.941371) (stroke (width 0.072) (type default)) (layer "Edge.Cuts"))
 (gr_line (start 94.946565 91.29143) (end 98.875569 90.787344) (stroke (width 0.072) (type default)) (layer "Edge.Cuts"))
 (gr_line (start 104.394632 94.206562) (end 104.419533 94.542612) (stroke (width 0.072) (type default)) (layer "Edge.Cuts"))
 (gr_line (start 93.346617 66.224835) (end 100.218585 75.003651) (stroke (width 0.072) (type default)) (layer "Edge.Cuts"))
 (gr_line (start 125.096741 88.844337) (end 126.158003 87.502729) (stroke (width 0.072) (type default)) (layer "Edge.Cuts"))
 (gr_line (start 122.041173 79.393912) (end 120.810207 78.895068) (stroke (width 0.072) (type default)) (layer "Edge.Cuts"))
 (gr_line (start 115.856243 89.457306) (end 116.573954 90.14983) (stroke (width 0.072) (type default)) (layer "Edge.Cuts"))
 (gr_line (start 95.857333 84.859764) (end 96.845417 85.284808) (stroke (width 0.072) (type default)) (layer "Edge.Cuts"))
 (gr_line (start 99.645177 96.359514) (end 101.045311 96.214005) (stroke (width 0.072) (type default)) (layer "Edge.Cuts"))
 (gr_line (start 98.208716 94.656213) (end 98.426372 95.050622) (stroke (width 0.072) (type default)) (layer "Edge.Cuts"))
 (gr_line (start 124.660868 94.1893) (end 124.927909 94.088853) (stroke (width 0.072) (type default)) (layer "Edge.Cuts"))
 (gr_line (start 91.775246 90.260232) (end 91.222185 90.665026) (stroke (width 0.072) (type default)) (layer "Edge.Cuts"))
 (gr_line (start 116.573954 90.14983) (end 120.542918 93.132459) (stroke (width 0.072) (type default)) (layer "Edge.Cuts"))
 (gr_line (start 93.515277 66.106532) (end 93.346617 66.224835) (stroke (width 0.072) (type default)) (layer "Edge.Cuts"))
 (gr_line (start 100.218585 75.003651) (end 100.645682 75.470046) (stroke (width 0.072) (type default)) (layer "Edge.Cuts"))
 (gr_line (start 92.622679 74.941371) (end 92.337541 75.228889) (stroke (width 0.072) (type default)) (layer "Edge.Cuts"))
 (gr_line (start 94.183192 84.047888) (end 95.857333 84.859764) (stroke (width 0.072) (type default)) (layer "Edge.Cuts"))
 (gr_line (start 93.087017 76.351333) (end 96.717751 79.919415) (stroke (width 0.072) (type default)) (layer "Edge.Cuts"))
 (gr_line (start 124.840403 80.129893) (end 123.327651 79.776042) (stroke (width 0.072) (type default)) (layer "Edge.Cuts"))
 (gr_line (start 104.54158 69.439941) (end 104.997221 70.380067) (stroke (width 0.072) (type default)) (layer "Edge.Cuts"))
 (gr_line (start 123.202094 93.410923) (end 123.804075 93.76949) (stroke (width 0.072) (type default)) (layer "Edge.Cuts"))
 (gr_line (start 123.184414 93.689401) (end 123.202094 93.410923) (stroke (width 0.072) (type default)) (layer "Edge.Cuts"))
 (gr_line (start 92.337541 75.228889) (end 93.087017 76.351333) (stroke (width 0.072) (type default)) (layer "Edge.Cuts"))
 (gr_line (start 98.426372 95.050622) (end 99.766094 93.854803) (stroke (width 0.072) (type default)) (layer "Edge.Cuts"))
 (gr_line (start 96.717751 79.919415) (end 97.936253 80.949577) (stroke (width 0.072) (type default)) (layer "Edge.Cuts"))
 (gr_line (start 120.542918 93.132459) (end 121.295109 93.415542) (stroke (width 0.072) (type default)) (layer "Edge.Cuts"))
 (gr_line (start 98.892698 91.495604) (end 98.208716 94.656213) (stroke (width 0.072) (type default)) (layer "Edge.Cuts"))
 (gr_line (start 101.045311 96.214005) (end 103.798875 94.675578) (stroke (width 0.072) (type default)) (layer "Edge.Cuts"))
 (gr_line (start 123.804075 93.76949) (end 124.660868 94.1893) (stroke (width 0.072) (type default)) (layer "Edge.Cuts"))
 (gr_line (start 91.431179 90.926584) (end 94.946565 91.29143) (stroke (width 0.072) (type default)) (layer "Edge.Cuts"))
 (gr_line (start 130.339223 83.843257) (end 124.840403 80.129893) (stroke (width 0.072) (type default)) (layer "Edge.Cuts"))
 (gr_line (start 120.021404 77.718346) (end 118.91188 76.005078) (stroke (width 0.072) (type default)) (layer "Edge.Cuts"))
 (gr_line (start 104.997221 70.380067) (end 105.156539 70.765324) (stroke (width 0.072) (type default)) (layer "Edge.Cuts"))
 (gr_line (start 107.513121 92.531871) (end 109.593507 91.025541) (stroke (width 0.072) (type default)) (layer "Edge.Cuts"))
 (gr_line (start 96.295917 66.996459) (end 93.515241 66.106532) (stroke (width 0.072) (type default)) (layer "Edge.Cuts"))
 (gr_line (start 103.798875 94.675578) (end 104.394632 94.206562) (stroke (width 0.072) (type default)) (layer "Edge.Cuts"))
 (gr_line (start 128.563837 85.821273) (end 130.339223 83.843257) (stroke (width 0.072) (type default)) (layer "Edge.Cuts"))
 (gr_line (start 126.158003 87.502729) (end 128.563837 85.821273) (stroke (width 0.072) (type default)) (layer "Edge.Cuts"))
 (gr_line (start 97.116307 81.268875) (end 93.196663 82.037306) (stroke (width 0.072) (type default)) (layer "Edge.Cuts"))
 (gr_line (start 105.479751 95.049837) (end 107.513121 92.531871) (stroke (width 0.072) (type default)) (layer "Edge.Cuts"))
 (gr_line (start 99.145429 90.714087) (end 98.892698 91.495604) (stroke (width 0.072) (type default)) (layer "Edge.Cuts"))
 (gr_line (start 104.419533 94.542612) (end 104.694058 95.977395) (stroke (width 0.072) (type default)) (layer "Edge.Cuts"))
 (gr_line (start 123.10862 94.035926) (end 123.184414 93.689401) (stroke (width 0.072) (type default)) (layer "Edge.Cuts"))
 (gr_line (start 99.766094 93.854803) (end 101.117966 92.679648) (stroke (width 0.072) (type default)) (layer "Edge.Cuts"))
 (gr_line (start 104.397829 68.617593) (end 104.54158 69.439941) (stroke (width 0.072) (type default)) (layer "Edge.Cuts"))
 (gr_line (start 91.222185 90.665026) (end 91.431179 90.926584) (stroke (width 0.072) (type default)) (layer "Edge.Cuts"))
 (gr_line (start 117.781603 74.75299) (end 111.378247 72.377552) (stroke (width 0.072) (type default)) (layer "Edge.Cuts"))
 (segment (start 103.825 89.3925) (end 103.5475 89.67) (width 0.2) (layer "B.Cu") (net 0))
 (segment (start 107.635 81.190552) (end 107.635 80.845) (width 0.2) (layer "B.Cu") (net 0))
 (segment (start 106.365 78.875) (end 106.365 80.845) (width 0.2) (layer "B.Cu") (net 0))
 (segment (start 105.095 79.870001) (end 104.734999 79.51) (width 0.2) (layer "B.Cu") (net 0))
 (segment (start 105.095 89.3925) (end 105.3725 89.67) (width 0.2) (layer "B.Cu") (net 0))
 (segment (start 106.365 85.795) (end 106.365 84.820001) (width 0.2) (layer "B.Cu") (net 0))
 (segment (start 105.095 85.795) (end 105.095 89.3925) (width 0.2) (layer "B.Cu") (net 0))
 (segment (start 100.65 81.8575) (end 99.38 83.1275) (width 0.2) (layer "B.Cu") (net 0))
 (segment (start 116.6175 78.7825) (end 115.89 79.51) (width 0.2) (layer "B.Cu") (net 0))
 (segment (start 110.81 86.065) (end 114.62 86.065) (width 0.2) (layer "B.Cu") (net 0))
 (segment (start 105.469744 91.07) (end 106.365 90.174744) (width 0.2) (layer "B.Cu") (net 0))
 (segment (start 105.095 80.845) (end 105.095 79.870001) (width 0.2) (layer "B.Cu") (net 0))
 (segment (start 107.635 80.845) (end 118.876 80.845) (width 0.2) (layer "B.Cu") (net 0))
 (segment (start 116.6175 77.08) (end 116.6175 78.7825) (width 0.2) (layer "B.Cu") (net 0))
 (segment (start 100.65 84.7825) (end 100.65 89.67) (width 0.2) (layer "B.Cu") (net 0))
 (segment (start 99.38 88.965686) (end 101.484314 91.07) (width 0.2) (layer "B.Cu") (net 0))
 (segment (start 104.734999 79.51) (end 102.9975 79.51) (width 0.2) (layer "B.Cu") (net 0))
 (segment (start 109.265 84.52) (end 110.81 86.065) (width 0.2) (layer "B.Cu") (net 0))
 (segment (start 100.65 89.67) (end 101.65 90.67) (width 0.2) (layer "B.Cu") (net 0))
 (segment (start 106.665001 84.52) (end 109.265 84.52) (width 0.2) (layer "B.Cu") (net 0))
 (segment (start 106.365 90.174744) (end 106.365 85.795) (width 0.2) (layer "B.Cu") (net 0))
 (segment (start 104.3725 90.67) (end 105.3725 89.67) (width 0.2) (layer "B.Cu") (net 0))
 (segment (start 114.7425 77.08) (end 108.16 77.08) (width 0.2) (layer "B.Cu") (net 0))
 (segment (start 99.38 83.1275) (end 99.38 88.965686) (width 0.2) (layer "B.Cu") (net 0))
 (segment (start 103.825 85.795) (end 103.825 89.3925) (width 0.2) (layer "B.Cu") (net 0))
 (segment (start 106.365 84.820001) (end 106.665001 84.52) (width 0.2) (layer "B.Cu") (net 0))
 (segment (start 103.825 85.000552) (end 107.635 81.190552) (width 0.2) (layer "B.Cu") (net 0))
 (segment (start 118.876 80.845) (end 120.97 82.939) (width 0.2) (layer "B.Cu") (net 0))
 (segment (start 102.9975 79.51) (end 100.65 81.8575) (width 0.2) (layer "B.Cu") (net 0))
 (segment (start 101.65 90.67) (end 104.3725 90.67) (width 0.2) (layer "B.Cu") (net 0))
 (segment (start 115.5975 79.2175) (end 115.89 79.51) (width 0.2) (layer "B.Cu") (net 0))
 (segment (start 108.16 77.08) (end 106.365 78.875) (width 0.2) (layer "B.Cu") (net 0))
 (segment (start 101.484314 91.07) (end 105.469744 91.07) (width 0.2) (layer "B.Cu") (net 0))
 (segment (start 103.825 85.795) (end 103.825 85.000552) (width 0.2) (layer "B.Cu") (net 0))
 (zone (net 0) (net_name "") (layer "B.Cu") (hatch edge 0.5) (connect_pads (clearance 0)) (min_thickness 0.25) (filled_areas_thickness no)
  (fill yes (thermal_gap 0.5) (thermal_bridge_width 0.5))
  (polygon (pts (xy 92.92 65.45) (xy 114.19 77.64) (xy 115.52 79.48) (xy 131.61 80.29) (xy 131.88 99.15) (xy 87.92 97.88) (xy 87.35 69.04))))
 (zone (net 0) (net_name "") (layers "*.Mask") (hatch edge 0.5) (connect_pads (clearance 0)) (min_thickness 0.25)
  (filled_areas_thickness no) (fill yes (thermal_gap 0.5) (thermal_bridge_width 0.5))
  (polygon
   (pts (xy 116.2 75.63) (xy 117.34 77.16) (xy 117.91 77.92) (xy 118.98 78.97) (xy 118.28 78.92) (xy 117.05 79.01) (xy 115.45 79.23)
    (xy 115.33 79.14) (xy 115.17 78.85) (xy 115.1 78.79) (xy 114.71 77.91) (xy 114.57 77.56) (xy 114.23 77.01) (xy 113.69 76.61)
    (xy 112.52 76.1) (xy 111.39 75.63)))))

